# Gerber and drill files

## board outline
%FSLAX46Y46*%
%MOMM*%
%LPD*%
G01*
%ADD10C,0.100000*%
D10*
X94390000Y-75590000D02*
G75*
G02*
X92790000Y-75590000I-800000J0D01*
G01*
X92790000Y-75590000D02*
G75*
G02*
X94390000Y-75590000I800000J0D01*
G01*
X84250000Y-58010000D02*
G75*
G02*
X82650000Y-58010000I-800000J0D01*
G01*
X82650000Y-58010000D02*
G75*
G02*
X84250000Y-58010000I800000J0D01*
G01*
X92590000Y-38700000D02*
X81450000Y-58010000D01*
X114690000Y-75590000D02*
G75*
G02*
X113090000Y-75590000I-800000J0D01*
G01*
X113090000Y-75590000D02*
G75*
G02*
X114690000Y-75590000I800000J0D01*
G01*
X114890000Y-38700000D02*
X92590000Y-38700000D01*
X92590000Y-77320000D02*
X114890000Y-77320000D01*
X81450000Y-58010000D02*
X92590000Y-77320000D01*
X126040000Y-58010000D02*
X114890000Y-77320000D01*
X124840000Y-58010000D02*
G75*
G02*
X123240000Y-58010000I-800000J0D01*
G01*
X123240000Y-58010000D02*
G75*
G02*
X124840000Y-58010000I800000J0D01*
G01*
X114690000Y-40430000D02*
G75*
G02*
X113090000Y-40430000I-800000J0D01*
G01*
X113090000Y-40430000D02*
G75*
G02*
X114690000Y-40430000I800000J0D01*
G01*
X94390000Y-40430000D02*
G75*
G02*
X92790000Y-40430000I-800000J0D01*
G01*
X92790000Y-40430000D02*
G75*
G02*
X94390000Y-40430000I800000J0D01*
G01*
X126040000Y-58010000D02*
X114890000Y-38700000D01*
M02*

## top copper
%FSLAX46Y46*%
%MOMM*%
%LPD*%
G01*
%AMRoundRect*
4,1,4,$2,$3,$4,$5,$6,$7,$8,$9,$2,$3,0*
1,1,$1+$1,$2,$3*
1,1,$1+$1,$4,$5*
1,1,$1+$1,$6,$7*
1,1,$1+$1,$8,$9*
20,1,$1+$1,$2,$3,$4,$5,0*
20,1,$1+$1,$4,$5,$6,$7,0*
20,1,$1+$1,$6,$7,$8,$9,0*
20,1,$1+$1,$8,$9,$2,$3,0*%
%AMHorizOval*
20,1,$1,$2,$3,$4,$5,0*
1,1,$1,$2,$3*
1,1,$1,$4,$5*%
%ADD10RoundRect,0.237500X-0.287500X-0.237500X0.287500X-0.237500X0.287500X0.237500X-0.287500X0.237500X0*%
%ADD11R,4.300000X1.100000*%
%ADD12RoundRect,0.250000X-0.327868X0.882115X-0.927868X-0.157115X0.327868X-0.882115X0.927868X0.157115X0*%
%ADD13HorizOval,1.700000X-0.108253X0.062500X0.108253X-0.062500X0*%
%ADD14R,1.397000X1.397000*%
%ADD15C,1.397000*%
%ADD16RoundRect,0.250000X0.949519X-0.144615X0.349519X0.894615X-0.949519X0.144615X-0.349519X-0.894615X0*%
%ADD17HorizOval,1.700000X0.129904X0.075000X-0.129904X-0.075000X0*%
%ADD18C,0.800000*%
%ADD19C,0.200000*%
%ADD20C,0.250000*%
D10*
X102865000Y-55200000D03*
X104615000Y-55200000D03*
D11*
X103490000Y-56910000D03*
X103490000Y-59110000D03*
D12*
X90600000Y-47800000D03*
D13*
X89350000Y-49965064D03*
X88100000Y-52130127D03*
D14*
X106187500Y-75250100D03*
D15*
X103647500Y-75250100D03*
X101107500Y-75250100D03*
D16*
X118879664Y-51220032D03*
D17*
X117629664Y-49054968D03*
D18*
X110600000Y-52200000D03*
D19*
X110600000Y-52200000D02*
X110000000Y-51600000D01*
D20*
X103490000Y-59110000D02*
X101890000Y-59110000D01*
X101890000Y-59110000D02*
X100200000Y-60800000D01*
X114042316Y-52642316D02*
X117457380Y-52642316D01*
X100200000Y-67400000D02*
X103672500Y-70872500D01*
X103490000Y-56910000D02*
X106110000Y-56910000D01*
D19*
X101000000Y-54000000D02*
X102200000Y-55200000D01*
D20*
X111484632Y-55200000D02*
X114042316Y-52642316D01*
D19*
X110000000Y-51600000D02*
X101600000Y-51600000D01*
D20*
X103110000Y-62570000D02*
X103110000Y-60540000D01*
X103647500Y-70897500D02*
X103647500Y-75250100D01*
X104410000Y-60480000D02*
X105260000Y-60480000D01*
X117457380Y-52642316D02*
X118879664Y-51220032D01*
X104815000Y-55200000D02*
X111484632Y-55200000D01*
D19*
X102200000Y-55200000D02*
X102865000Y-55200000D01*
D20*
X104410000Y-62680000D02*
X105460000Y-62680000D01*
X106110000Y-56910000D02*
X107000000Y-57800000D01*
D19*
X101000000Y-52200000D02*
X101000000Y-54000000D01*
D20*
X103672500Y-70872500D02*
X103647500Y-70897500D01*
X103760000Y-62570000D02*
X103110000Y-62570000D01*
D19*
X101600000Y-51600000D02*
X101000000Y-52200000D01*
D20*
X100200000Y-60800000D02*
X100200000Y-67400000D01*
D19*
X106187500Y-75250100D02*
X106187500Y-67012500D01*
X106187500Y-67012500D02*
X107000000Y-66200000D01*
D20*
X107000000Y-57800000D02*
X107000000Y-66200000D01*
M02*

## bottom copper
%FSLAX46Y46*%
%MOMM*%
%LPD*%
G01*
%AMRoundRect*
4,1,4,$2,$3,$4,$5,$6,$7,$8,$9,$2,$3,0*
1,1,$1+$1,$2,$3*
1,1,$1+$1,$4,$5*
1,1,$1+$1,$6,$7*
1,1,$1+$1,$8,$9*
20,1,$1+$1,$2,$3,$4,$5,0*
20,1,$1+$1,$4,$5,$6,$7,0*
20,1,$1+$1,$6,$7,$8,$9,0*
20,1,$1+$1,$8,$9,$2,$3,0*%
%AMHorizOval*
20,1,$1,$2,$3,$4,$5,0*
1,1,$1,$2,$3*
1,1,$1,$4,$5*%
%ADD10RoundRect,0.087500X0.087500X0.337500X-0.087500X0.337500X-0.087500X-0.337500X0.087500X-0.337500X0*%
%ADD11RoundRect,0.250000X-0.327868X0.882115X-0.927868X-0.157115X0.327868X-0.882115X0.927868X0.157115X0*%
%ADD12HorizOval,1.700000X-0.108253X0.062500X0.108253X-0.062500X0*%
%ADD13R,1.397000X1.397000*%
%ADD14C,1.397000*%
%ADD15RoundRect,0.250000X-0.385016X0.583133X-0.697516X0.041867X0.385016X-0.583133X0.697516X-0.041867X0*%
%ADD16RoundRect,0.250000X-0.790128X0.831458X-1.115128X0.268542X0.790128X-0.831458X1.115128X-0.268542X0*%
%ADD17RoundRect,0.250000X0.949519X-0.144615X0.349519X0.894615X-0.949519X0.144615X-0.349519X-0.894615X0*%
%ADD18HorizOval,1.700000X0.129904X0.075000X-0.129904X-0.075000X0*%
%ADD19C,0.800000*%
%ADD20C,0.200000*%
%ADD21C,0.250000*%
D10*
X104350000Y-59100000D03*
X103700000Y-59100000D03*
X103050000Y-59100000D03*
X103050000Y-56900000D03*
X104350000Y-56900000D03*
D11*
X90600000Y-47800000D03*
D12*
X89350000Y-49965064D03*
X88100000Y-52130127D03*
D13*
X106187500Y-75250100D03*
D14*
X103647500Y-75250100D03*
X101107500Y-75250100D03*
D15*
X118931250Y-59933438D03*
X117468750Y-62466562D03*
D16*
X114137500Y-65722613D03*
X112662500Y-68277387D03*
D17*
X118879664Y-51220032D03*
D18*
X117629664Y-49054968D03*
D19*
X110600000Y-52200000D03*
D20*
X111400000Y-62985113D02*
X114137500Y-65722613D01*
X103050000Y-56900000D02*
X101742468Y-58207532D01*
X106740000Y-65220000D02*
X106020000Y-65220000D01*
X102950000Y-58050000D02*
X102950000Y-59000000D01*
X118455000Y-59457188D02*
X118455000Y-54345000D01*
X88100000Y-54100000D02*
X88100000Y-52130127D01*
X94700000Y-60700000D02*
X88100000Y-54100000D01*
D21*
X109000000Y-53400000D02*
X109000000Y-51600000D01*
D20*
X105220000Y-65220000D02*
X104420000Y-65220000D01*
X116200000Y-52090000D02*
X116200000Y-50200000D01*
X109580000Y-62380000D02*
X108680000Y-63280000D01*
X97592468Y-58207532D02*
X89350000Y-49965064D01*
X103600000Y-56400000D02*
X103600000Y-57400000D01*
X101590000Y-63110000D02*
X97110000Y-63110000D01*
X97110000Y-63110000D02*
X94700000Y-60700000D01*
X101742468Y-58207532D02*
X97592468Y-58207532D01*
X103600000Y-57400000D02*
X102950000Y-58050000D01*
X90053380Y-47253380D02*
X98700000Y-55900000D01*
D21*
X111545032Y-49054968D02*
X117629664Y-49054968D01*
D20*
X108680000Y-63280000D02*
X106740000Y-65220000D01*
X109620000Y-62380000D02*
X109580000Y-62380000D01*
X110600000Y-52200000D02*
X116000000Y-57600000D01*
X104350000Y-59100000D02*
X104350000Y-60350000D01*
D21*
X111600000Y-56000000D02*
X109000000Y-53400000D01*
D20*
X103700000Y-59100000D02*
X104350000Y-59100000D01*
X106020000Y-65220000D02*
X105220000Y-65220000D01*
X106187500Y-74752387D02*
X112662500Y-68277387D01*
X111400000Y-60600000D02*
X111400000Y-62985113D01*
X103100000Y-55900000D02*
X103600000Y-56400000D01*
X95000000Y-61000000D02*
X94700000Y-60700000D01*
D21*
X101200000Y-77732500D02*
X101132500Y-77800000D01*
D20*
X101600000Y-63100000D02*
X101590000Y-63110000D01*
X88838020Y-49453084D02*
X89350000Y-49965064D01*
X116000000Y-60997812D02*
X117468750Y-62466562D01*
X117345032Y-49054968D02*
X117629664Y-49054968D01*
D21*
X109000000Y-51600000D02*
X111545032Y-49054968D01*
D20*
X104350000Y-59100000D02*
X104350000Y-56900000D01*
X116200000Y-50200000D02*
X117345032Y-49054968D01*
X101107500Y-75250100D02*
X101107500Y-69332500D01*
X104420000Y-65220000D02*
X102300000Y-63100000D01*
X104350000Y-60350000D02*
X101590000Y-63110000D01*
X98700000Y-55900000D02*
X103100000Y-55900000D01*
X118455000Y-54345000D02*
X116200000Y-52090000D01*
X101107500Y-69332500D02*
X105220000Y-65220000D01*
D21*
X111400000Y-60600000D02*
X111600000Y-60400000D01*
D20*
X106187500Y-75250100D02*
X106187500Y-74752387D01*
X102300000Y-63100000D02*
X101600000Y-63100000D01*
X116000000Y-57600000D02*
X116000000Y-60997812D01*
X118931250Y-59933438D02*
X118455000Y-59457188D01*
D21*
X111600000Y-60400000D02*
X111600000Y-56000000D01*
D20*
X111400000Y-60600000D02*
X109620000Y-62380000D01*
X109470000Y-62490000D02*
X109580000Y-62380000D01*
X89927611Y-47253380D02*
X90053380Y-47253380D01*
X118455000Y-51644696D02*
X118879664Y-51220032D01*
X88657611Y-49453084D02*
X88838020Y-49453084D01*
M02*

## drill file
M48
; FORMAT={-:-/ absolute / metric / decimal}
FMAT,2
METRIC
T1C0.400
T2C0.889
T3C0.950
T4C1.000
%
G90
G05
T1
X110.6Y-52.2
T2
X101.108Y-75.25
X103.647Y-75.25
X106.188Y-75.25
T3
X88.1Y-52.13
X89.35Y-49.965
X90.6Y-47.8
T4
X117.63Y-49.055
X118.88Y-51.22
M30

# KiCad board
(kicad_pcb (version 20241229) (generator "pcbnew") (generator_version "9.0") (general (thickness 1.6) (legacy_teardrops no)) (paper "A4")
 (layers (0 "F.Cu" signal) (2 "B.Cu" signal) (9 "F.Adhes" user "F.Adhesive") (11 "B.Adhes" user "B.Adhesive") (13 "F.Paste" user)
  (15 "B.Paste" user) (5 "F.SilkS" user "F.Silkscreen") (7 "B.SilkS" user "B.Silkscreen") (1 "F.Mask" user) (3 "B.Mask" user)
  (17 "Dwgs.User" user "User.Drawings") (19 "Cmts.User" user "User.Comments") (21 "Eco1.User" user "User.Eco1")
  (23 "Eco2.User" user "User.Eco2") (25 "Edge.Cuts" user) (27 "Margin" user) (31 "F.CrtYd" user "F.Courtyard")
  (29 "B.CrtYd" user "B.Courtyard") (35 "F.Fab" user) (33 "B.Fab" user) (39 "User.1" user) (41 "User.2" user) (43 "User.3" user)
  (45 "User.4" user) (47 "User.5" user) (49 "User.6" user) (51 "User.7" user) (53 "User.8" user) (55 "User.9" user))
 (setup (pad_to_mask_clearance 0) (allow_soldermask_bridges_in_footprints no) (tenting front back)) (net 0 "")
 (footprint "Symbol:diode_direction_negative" (layer "F.Cu") (at 103.8 52.65)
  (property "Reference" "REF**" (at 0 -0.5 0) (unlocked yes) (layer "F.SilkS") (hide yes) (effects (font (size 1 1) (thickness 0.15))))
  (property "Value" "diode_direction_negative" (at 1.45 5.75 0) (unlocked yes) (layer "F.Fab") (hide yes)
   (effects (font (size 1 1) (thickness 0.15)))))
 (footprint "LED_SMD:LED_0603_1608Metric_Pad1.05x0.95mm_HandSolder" (layer "F.Cu") (at 103.74 55.2)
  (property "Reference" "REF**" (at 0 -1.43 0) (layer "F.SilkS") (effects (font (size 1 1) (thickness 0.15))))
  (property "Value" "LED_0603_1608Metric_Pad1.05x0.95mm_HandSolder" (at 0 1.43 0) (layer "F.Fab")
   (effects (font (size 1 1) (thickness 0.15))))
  (pad "1" smd roundrect (at -0.875 0) (size 1.05 0.95) (layers "F.Cu" "F.Mask" "F.Paste") (roundrect_rratio 0.25))
  (pad "2" smd roundrect (at 0.875 0) (size 1.05 0.95) (layers "F.Cu" "F.Mask" "F.Paste") (roundrect_rratio 0.25)))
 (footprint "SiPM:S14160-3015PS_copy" (layer "F.Cu") (at 103.74 58.01)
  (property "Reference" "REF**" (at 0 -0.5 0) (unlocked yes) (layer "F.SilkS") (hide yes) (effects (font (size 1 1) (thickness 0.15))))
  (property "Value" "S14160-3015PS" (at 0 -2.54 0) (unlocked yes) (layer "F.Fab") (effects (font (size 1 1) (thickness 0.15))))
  (pad "1" smd rect (at -0.25 -1.1) (size 4.3 1.1) (layers "F.Cu" "F.Mask" "F.Paste"))
  (pad "2" smd rect (at -0.25 1.1) (size 4.3 1.1) (layers "F.Cu" "F.Mask" "F.Paste")))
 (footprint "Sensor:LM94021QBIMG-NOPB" (layer "B.Cu") (at 103.7 58 180)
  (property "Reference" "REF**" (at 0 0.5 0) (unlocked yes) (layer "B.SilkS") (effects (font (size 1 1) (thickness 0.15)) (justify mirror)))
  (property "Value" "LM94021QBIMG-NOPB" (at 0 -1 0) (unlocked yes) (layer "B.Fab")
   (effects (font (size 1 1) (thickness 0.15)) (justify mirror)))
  (pad "1" smd roundrect (at -0.65 -1.1 180) (size 0.35 0.85) (layers "B.Cu" "B.Mask" "B.Paste") (roundrect_rratio 0.25))
  (pad "2" smd roundrect (at 0 -1.1 180) (size 0.35 0.85) (layers "B.Cu" "B.Mask" "B.Paste") (roundrect_rratio 0.25))
  (pad "3" smd roundrect (at 0.65 -1.1 180) (size 0.35 0.85) (layers "B.Cu" "B.Mask" "B.Paste") (roundrect_rratio 0.25))
  (pad "4" smd roundrect (at 0.65 1.1 180) (size 0.35 0.85) (layers "B.Cu" "B.Mask" "B.Paste") (roundrect_rratio 0.25))
  (pad "5" smd roundrect (at -0.65 1.1 180) (size 0.35 0.85) (layers "B.Cu" "B.Mask" "B.Paste") (roundrect_rratio 0.25)))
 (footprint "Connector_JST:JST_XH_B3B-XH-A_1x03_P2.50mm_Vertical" (layer "B.Cu") (at 90.6 47.8 -120)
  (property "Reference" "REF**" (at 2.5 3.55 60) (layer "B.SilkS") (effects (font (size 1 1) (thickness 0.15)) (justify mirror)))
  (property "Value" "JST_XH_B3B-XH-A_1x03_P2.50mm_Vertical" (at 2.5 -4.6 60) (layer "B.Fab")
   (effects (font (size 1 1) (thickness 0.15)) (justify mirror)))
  (pad "1" thru_hole roundrect (at 0 0 240) (size 1.7 1.95) (drill 0.95) (layers "*.Cu" "*.Mask") (remove_unused_layers no)
   (roundrect_rratio 0.1470588235))
  (pad "2" thru_hole oval (at 2.5 0 240) (size 1.7 1.95) (drill 0.95) (layers "*.Cu" "*.Mask") (remove_unused_layers no))
  (pad "3" thru_hole oval (at 5 0 240) (size 1.7 1.95) (drill 0.95) (layers "*.Cu" "*.Mask") (remove_unused_layers no)))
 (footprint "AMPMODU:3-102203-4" (layer "B.Cu") (at 106.1875 75.2501 180)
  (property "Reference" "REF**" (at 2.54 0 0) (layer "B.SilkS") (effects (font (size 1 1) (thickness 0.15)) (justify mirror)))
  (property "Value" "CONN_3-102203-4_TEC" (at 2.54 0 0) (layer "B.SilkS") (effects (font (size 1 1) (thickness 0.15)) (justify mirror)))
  (pad "1" thru_hole rect (at 0 0 180) (size 1.397 1.397) (drill 0.889) (layers "*.Cu" "*.Mask") (remove_unused_layers no))
  (pad "2" thru_hole circle (at 2.54 0 180) (size 1.397 1.397) (drill 0.889) (layers "*.Cu" "*.Mask") (remove_unused_layers no))
  (pad "3" thru_hole circle (at 5.08 0 180) (size 1.397 1.397) (drill 0.889) (layers "*.Cu" "*.Mask") (remove_unused_layers no)))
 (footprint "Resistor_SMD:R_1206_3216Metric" (layer "B.Cu") (at 118.2 61.2 -120)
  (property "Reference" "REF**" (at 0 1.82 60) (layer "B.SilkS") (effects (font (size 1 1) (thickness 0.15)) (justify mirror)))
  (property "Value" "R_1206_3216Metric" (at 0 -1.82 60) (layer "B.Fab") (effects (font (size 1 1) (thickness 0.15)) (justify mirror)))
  (pad "1" smd roundrect (at -1.4625 0 240) (size 1.125 1.75) (layers "B.Cu" "B.Mask" "B.Paste") (roundrect_rratio 0.222222))
  (pad "2" smd roundrect (at 1.4625 0 240) (size 1.125 1.75) (layers "B.Cu" "B.Mask" "B.Paste") (roundrect_rratio 0.222222)))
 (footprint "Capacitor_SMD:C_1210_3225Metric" (layer "B.Cu") (at 113.4 67 -120)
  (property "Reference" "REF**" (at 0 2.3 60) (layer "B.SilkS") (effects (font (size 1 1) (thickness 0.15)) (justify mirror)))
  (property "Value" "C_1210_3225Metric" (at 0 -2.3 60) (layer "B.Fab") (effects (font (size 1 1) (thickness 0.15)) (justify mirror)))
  (pad "1" smd roundrect (at -1.475 0 240) (size 1.15 2.7) (layers "B.Cu" "B.Mask" "B.Paste") (roundrect_rratio 0.2173913043))
  (pad "2" smd roundrect (at 1.475 0 240) (size 1.15 2.7) (layers "B.Cu" "B.Mask" "B.Paste") (roundrect_rratio 0.2173913043)))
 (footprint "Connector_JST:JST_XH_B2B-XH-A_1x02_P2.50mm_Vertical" (layer "B.Cu") (at 118.879664 51.220032 120)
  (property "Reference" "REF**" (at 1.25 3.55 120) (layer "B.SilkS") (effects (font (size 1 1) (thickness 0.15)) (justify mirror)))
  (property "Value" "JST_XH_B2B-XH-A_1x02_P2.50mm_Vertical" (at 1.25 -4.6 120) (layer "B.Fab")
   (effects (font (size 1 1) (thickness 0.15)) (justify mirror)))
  (pad "1" thru_hole roundrect (at 0 0 120) (size 1.7 2) (drill 1) (layers "*.Cu" "*.Mask") (remove_unused_layers no)
   (roundrect_rratio 0.1470588235))
  (pad "2" thru_hole oval (at 2.5 0 120) (size 1.7 2) (drill 1) (layers "*.Cu" "*.Mask") (remove_unused_layers no)))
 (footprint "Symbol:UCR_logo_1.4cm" (layer "B.Cu") (at 104.4 43 180)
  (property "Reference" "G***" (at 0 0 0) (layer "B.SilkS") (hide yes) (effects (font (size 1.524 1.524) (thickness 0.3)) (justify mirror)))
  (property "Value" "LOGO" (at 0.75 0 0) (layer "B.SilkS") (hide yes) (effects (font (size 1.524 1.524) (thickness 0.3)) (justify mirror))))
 (gr_circle (center 93.59 75.59) (end 94.39 75.59) (stroke (width 0.1) (type solid)) (fill no) (layer "Edge.Cuts"))
 (gr_circle (center 83.45 58.01) (end 84.25 58.01) (stroke (width 0.1) (type solid)) (fill no) (layer "Edge.Cuts"))
 (gr_line (start 92.59 38.7) (end 81.45 58.01) (stroke (width 0.1) (type solid)) (layer "Edge.Cuts"))
 (gr_circle (center 113.89 75.59) (end 114.69 75.59) (stroke (width 0.1) (type solid)) (fill no) (layer "Edge.Cuts"))
 (gr_line (start 114.89 38.7) (end 92.59 38.7) (stroke (width 0.1) (type solid)) (layer "Edge.Cuts"))
 (gr_line (start 92.59 77.32) (end 114.89 77.32) (stroke (width 0.1) (type solid)) (layer "Edge.Cuts"))
 (gr_line (start 81.45 58.01) (end 92.59 77.32) (stroke (width 0.1) (type solid)) (layer "Edge.Cuts"))
 (gr_line (start 126.04 58.01) (end 114.89 77.32) (stroke (width 0.1) (type solid)) (layer "Edge.Cuts"))
 (gr_circle (center 124.04 58.01) (end 124.84 58.01) (stroke (width 0.1) (type solid)) (fill no) (layer "Edge.Cuts"))
 (gr_circle (center 113.89 40.43) (end 114.69 40.43) (stroke (width 0.1) (type solid)) (fill no) (layer "Edge.Cuts"))
 (gr_circle (center 93.59 40.43) (end 94.39 40.43) (stroke (width 0.1) (type solid)) (fill no) (layer "Edge.Cuts"))
 (gr_line (start 126.04 58.01) (end 114.89 38.7) (stroke (width 0.1) (type solid)) (layer "Edge.Cuts"))
 (segment (start 110.6 52.2) (end 110 51.6) (width 0.2) (layer "F.Cu") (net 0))
 (segment (start 103.49 59.11) (end 101.89 59.11) (width 0.25) (layer "F.Cu") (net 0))
 (segment (start 101.89 59.11) (end 100.2 60.8) (width 0.25) (layer "F.Cu") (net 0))
 (segment (start 114.042316 52.642316) (end 117.45738 52.642316) (width 0.25) (layer "F.Cu") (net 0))
 (segment (start 100.2 67.4) (end 103.6725 70.8725) (width 0.25) (layer "F.Cu") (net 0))
 (segment (start 103.49 56.91) (end 106.11 56.91) (width 0.25) (layer "F.Cu") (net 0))
 (segment (start 101 54) (end 102.2 55.2) (width 0.2) (layer "F.Cu") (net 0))
 (segment (start 111.484632 55.2) (end 114.042316 52.642316) (width 0.25) (layer "F.Cu") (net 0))
 (segment (start 110 51.6) (end 101.6 51.6) (width 0.2) (layer "F.Cu") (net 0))
 (segment (start 103.11 62.57) (end 103.11 60.54) (width 0.25) (layer "F.Cu") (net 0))
 (segment (start 103.6475 70.8975) (end 103.6475 75.2501) (width 0.25) (layer "F.Cu") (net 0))
 (segment (start 104.41 60.48) (end 105.26 60.48) (width 0.25) (layer "F.Cu") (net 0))
 (segment (start 117.45738 52.642316) (end 118.879664 51.220032) (width 0.25) (layer "F.Cu") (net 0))
 (segment (start 104.815 55.2) (end 111.484632 55.2) (width 0.25) (layer "F.Cu") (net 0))
 (segment (start 102.2 55.2) (end 102.865 55.2) (width 0.2) (layer "F.Cu") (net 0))
 (segment (start 104.41 62.68) (end 105.46 62.68) (width 0.25) (layer "F.Cu") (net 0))
 (segment (start 106.11 56.91) (end 107 57.8) (width 0.25) (layer "F.Cu") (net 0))
 (segment (start 101 52.2) (end 101 54) (width 0.2) (layer "F.Cu") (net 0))
 (segment (start 103.6725 70.8725) (end 103.6475 70.8975) (width 0.25) (layer "F.Cu") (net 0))
 (segment (start 103.76 62.57) (end 103.11 62.57) (width 0.25) (layer "F.Cu") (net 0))
 (segment (start 101.6 51.6) (end 101 52.2) (width 0.2) (layer "F.Cu") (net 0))
 (segment (start 100.2 60.8) (end 100.2 67.4) (width 0.25) (layer "F.Cu") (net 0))
 (segment (start 106.1875 75.2501) (end 106.1875 67.0125) (width 0.2) (layer "F.Cu") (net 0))
 (segment (start 106.1875 67.0125) (end 107 66.2) (width 0.2) (layer "F.Cu") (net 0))
 (segment (start 107 57.8) (end 107 66.2) (width 0.25) (layer "F.Cu") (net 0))
 (via (at 110.6 52.2) (size 0.8) (drill 0.4) (layers "F.Cu" "B.Cu") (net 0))
 (segment (start 111.4 62.985113) (end 114.1375 65.722613) (width 0.2) (layer "B.Cu") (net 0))
 (segment (start 103.05 56.9) (end 101.742468 58.207532) (width 0.2) (layer "B.Cu") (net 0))
 (segment (start 106.74 65.22) (end 106.02 65.22) (width 0.2) (layer "B.Cu") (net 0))
 (segment (start 102.95 58.05) (end 102.95 59) (width 0.2) (layer "B.Cu") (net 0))
 (segment (start 118.455 59.457188) (end 118.455 54.345) (width 0.2) (layer "B.Cu") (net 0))
 (segment (start 88.1 54.1) (end 88.1 52.130127) (width 0.2) (layer "B.Cu") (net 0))
 (segment (start 94.7 60.7) (end 88.1 54.1) (width 0.2) (layer "B.Cu") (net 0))
 (segment (start 109 53.4) (end 109 51.6) (width 0.25) (layer "B.Cu") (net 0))
 (segment (start 105.22 65.22) (end 104.42 65.22) (width 0.2) (layer "B.Cu") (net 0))
 (segment (start 116.2 52.09) (end 116.2 50.2) (width 0.2) (layer "B.Cu") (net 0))
 (segment (start 109.58 62.38) (end 108.68 63.28) (width 0.2) (layer "B.Cu") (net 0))
 (segment (start 97.592468 58.207532) (end 89.35 49.965064) (width 0.2) (layer "B.Cu") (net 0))
 (segment (start 103.6 56.4) (end 103.6 57.4) (width 0.2) (layer "B.Cu") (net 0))
 (segment (start 101.59 63.11) (end 97.11 63.11) (width 0.2) (layer "B.Cu") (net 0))
 (segment (start 97.11 63.11) (end 94.7 60.7) (width 0.2) (layer "B.Cu") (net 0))
 (segment (start 101.742468 58.207532) (end 97.592468 58.207532) (width 0.2) (layer "B.Cu") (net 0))
 (segment (start 103.6 57.4) (end 102.95 58.05) (width 0.2) (layer "B.Cu") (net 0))
 (segment (start 90.05338 47.25338) (end 98.7 55.9) (width 0.2) (layer "B.Cu") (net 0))
 (segment (start 111.545032 49.054968) (end 117.629664 49.054968) (width 0.25) (layer "B.Cu") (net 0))
 (segment (start 108.68 63.28) (end 106.74 65.22) (width 0.2) (layer "B.Cu") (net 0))
 (segment (start 109.62 62.38) (end 109.58 62.38) (width 0.2) (layer "B.Cu") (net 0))
 (segment (start 110.6 52.2) (end 116 57.6) (width 0.2) (layer "B.Cu") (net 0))
 (segment (start 104.35 59.1) (end 104.35 60.35) (width 0.2) (layer "B.Cu") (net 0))
 (segment (start 111.6 56) (end 109 53.4) (width 0.25) (layer "B.Cu") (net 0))
 (segment (start 103.7 59.1) (end 104.35 59.1) (width 0.2) (layer "B.Cu") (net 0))
 (segment (start 106.02 65.22) (end 105.22 65.22) (width 0.2) (layer "B.Cu") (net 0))
 (segment (start 106.1875 74.752387) (end 112.6625 68.277387) (width 0.2) (layer "B.Cu") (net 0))
 (segment (start 111.4 60.6) (end 111.4 62.985113) (width 0.2) (layer "B.Cu") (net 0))
 (segment (start 103.1 55.9) (end 103.6 56.4) (width 0.2) (layer "B.Cu") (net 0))
 (segment (start 95 61) (end 94.7 60.7) (width 0.2) (layer "B.Cu") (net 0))
 (segment (start 101.2 77.7325) (end 101.1325 77.8) (width 0.25) (layer "B.Cu") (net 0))
 (segment (start 101.6 63.1) (end 101.59 63.11) (width 0.2) (layer "B.Cu") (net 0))
 (segment (start 88.83802 49.453084) (end 89.35 49.965064) (width 0.2) (layer "B.Cu") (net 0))
 (segment (start 116 60.997812) (end 117.46875 62.466562) (width 0.2) (layer "B.Cu") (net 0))
 (segment (start 117.345032 49.054968) (end 117.629664 49.054968) (width 0.2) (layer "B.Cu") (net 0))
 (segment (start 109 51.6) (end 111.545032 49.054968) (width 0.25) (layer "B.Cu") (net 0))
 (segment (start 104.35 59.1) (end 104.35 56.9) (width 0.2) (layer "B.Cu") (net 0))
 (segment (start 116.2 50.2) (end 117.345032 49.054968) (width 0.2) (layer "B.Cu") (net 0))
 (segment (start 101.1075 75.2501) (end 101.1075 69.3325) (width 0.2) (layer "B.Cu") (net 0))
 (segment (start 104.42 65.22) (end 102.3 63.1) (width 0.2) (layer "B.Cu") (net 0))
 (segment (start 104.35 60.35) (end 101.59 63.11) (width 0.2) (layer "B.Cu") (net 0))
 (segment (start 98.7 55.9) (end 103.1 55.9) (width 0.2) (layer "B.Cu") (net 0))
 (segment (start 118.455 54.345) (end 116.2 52.09) (width 0.2) (layer "B.Cu") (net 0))
 (segment (start 101.1075 69.3325) (end 105.22 65.22) (width 0.2) (layer "B.Cu") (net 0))
 (segment (start 111.4 60.6) (end 111.6 60.4) (width 0.25) (layer "B.Cu") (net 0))
 (segment (start 106.1875 75.2501) (end 106.1875 74.752387) (width 0.2) (layer "B.Cu") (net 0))
 (segment (start 102.3 63.1) (end 101.6 63.1) (width 0.2) (layer "B.Cu") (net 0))
 (segment (start 116 57.6) (end 116 60.997812) (width 0.2) (layer "B.Cu") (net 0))
 (segment (start 118.93125 59.933438) (end 118.455 59.457188) (width 0.2) (layer "B.Cu") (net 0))
 (segment (start 111.6 60.4) (end 111.6 56) (width 0.25) (layer "B.Cu") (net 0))
 (segment (start 111.4 60.6) (end 109.62 62.38) (width 0.2) (layer "B.Cu") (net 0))
 (segment (start 109.47 62.49) (end 109.58 62.38) (width 0.2) (layer "B.Cu") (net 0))
 (segment (start 89.927611 47.25338) (end 90.05338 47.25338) (width 0.2) (layer "B.Cu") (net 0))
 (segment (start 118.455 51.644696) (end 118.879664 51.220032) (width 0.2) (layer "B.Cu") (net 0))
 (segment (start 88.657611 49.453084) (end 88.83802 49.453084) (width 0.2) (layer "B.Cu") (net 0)))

